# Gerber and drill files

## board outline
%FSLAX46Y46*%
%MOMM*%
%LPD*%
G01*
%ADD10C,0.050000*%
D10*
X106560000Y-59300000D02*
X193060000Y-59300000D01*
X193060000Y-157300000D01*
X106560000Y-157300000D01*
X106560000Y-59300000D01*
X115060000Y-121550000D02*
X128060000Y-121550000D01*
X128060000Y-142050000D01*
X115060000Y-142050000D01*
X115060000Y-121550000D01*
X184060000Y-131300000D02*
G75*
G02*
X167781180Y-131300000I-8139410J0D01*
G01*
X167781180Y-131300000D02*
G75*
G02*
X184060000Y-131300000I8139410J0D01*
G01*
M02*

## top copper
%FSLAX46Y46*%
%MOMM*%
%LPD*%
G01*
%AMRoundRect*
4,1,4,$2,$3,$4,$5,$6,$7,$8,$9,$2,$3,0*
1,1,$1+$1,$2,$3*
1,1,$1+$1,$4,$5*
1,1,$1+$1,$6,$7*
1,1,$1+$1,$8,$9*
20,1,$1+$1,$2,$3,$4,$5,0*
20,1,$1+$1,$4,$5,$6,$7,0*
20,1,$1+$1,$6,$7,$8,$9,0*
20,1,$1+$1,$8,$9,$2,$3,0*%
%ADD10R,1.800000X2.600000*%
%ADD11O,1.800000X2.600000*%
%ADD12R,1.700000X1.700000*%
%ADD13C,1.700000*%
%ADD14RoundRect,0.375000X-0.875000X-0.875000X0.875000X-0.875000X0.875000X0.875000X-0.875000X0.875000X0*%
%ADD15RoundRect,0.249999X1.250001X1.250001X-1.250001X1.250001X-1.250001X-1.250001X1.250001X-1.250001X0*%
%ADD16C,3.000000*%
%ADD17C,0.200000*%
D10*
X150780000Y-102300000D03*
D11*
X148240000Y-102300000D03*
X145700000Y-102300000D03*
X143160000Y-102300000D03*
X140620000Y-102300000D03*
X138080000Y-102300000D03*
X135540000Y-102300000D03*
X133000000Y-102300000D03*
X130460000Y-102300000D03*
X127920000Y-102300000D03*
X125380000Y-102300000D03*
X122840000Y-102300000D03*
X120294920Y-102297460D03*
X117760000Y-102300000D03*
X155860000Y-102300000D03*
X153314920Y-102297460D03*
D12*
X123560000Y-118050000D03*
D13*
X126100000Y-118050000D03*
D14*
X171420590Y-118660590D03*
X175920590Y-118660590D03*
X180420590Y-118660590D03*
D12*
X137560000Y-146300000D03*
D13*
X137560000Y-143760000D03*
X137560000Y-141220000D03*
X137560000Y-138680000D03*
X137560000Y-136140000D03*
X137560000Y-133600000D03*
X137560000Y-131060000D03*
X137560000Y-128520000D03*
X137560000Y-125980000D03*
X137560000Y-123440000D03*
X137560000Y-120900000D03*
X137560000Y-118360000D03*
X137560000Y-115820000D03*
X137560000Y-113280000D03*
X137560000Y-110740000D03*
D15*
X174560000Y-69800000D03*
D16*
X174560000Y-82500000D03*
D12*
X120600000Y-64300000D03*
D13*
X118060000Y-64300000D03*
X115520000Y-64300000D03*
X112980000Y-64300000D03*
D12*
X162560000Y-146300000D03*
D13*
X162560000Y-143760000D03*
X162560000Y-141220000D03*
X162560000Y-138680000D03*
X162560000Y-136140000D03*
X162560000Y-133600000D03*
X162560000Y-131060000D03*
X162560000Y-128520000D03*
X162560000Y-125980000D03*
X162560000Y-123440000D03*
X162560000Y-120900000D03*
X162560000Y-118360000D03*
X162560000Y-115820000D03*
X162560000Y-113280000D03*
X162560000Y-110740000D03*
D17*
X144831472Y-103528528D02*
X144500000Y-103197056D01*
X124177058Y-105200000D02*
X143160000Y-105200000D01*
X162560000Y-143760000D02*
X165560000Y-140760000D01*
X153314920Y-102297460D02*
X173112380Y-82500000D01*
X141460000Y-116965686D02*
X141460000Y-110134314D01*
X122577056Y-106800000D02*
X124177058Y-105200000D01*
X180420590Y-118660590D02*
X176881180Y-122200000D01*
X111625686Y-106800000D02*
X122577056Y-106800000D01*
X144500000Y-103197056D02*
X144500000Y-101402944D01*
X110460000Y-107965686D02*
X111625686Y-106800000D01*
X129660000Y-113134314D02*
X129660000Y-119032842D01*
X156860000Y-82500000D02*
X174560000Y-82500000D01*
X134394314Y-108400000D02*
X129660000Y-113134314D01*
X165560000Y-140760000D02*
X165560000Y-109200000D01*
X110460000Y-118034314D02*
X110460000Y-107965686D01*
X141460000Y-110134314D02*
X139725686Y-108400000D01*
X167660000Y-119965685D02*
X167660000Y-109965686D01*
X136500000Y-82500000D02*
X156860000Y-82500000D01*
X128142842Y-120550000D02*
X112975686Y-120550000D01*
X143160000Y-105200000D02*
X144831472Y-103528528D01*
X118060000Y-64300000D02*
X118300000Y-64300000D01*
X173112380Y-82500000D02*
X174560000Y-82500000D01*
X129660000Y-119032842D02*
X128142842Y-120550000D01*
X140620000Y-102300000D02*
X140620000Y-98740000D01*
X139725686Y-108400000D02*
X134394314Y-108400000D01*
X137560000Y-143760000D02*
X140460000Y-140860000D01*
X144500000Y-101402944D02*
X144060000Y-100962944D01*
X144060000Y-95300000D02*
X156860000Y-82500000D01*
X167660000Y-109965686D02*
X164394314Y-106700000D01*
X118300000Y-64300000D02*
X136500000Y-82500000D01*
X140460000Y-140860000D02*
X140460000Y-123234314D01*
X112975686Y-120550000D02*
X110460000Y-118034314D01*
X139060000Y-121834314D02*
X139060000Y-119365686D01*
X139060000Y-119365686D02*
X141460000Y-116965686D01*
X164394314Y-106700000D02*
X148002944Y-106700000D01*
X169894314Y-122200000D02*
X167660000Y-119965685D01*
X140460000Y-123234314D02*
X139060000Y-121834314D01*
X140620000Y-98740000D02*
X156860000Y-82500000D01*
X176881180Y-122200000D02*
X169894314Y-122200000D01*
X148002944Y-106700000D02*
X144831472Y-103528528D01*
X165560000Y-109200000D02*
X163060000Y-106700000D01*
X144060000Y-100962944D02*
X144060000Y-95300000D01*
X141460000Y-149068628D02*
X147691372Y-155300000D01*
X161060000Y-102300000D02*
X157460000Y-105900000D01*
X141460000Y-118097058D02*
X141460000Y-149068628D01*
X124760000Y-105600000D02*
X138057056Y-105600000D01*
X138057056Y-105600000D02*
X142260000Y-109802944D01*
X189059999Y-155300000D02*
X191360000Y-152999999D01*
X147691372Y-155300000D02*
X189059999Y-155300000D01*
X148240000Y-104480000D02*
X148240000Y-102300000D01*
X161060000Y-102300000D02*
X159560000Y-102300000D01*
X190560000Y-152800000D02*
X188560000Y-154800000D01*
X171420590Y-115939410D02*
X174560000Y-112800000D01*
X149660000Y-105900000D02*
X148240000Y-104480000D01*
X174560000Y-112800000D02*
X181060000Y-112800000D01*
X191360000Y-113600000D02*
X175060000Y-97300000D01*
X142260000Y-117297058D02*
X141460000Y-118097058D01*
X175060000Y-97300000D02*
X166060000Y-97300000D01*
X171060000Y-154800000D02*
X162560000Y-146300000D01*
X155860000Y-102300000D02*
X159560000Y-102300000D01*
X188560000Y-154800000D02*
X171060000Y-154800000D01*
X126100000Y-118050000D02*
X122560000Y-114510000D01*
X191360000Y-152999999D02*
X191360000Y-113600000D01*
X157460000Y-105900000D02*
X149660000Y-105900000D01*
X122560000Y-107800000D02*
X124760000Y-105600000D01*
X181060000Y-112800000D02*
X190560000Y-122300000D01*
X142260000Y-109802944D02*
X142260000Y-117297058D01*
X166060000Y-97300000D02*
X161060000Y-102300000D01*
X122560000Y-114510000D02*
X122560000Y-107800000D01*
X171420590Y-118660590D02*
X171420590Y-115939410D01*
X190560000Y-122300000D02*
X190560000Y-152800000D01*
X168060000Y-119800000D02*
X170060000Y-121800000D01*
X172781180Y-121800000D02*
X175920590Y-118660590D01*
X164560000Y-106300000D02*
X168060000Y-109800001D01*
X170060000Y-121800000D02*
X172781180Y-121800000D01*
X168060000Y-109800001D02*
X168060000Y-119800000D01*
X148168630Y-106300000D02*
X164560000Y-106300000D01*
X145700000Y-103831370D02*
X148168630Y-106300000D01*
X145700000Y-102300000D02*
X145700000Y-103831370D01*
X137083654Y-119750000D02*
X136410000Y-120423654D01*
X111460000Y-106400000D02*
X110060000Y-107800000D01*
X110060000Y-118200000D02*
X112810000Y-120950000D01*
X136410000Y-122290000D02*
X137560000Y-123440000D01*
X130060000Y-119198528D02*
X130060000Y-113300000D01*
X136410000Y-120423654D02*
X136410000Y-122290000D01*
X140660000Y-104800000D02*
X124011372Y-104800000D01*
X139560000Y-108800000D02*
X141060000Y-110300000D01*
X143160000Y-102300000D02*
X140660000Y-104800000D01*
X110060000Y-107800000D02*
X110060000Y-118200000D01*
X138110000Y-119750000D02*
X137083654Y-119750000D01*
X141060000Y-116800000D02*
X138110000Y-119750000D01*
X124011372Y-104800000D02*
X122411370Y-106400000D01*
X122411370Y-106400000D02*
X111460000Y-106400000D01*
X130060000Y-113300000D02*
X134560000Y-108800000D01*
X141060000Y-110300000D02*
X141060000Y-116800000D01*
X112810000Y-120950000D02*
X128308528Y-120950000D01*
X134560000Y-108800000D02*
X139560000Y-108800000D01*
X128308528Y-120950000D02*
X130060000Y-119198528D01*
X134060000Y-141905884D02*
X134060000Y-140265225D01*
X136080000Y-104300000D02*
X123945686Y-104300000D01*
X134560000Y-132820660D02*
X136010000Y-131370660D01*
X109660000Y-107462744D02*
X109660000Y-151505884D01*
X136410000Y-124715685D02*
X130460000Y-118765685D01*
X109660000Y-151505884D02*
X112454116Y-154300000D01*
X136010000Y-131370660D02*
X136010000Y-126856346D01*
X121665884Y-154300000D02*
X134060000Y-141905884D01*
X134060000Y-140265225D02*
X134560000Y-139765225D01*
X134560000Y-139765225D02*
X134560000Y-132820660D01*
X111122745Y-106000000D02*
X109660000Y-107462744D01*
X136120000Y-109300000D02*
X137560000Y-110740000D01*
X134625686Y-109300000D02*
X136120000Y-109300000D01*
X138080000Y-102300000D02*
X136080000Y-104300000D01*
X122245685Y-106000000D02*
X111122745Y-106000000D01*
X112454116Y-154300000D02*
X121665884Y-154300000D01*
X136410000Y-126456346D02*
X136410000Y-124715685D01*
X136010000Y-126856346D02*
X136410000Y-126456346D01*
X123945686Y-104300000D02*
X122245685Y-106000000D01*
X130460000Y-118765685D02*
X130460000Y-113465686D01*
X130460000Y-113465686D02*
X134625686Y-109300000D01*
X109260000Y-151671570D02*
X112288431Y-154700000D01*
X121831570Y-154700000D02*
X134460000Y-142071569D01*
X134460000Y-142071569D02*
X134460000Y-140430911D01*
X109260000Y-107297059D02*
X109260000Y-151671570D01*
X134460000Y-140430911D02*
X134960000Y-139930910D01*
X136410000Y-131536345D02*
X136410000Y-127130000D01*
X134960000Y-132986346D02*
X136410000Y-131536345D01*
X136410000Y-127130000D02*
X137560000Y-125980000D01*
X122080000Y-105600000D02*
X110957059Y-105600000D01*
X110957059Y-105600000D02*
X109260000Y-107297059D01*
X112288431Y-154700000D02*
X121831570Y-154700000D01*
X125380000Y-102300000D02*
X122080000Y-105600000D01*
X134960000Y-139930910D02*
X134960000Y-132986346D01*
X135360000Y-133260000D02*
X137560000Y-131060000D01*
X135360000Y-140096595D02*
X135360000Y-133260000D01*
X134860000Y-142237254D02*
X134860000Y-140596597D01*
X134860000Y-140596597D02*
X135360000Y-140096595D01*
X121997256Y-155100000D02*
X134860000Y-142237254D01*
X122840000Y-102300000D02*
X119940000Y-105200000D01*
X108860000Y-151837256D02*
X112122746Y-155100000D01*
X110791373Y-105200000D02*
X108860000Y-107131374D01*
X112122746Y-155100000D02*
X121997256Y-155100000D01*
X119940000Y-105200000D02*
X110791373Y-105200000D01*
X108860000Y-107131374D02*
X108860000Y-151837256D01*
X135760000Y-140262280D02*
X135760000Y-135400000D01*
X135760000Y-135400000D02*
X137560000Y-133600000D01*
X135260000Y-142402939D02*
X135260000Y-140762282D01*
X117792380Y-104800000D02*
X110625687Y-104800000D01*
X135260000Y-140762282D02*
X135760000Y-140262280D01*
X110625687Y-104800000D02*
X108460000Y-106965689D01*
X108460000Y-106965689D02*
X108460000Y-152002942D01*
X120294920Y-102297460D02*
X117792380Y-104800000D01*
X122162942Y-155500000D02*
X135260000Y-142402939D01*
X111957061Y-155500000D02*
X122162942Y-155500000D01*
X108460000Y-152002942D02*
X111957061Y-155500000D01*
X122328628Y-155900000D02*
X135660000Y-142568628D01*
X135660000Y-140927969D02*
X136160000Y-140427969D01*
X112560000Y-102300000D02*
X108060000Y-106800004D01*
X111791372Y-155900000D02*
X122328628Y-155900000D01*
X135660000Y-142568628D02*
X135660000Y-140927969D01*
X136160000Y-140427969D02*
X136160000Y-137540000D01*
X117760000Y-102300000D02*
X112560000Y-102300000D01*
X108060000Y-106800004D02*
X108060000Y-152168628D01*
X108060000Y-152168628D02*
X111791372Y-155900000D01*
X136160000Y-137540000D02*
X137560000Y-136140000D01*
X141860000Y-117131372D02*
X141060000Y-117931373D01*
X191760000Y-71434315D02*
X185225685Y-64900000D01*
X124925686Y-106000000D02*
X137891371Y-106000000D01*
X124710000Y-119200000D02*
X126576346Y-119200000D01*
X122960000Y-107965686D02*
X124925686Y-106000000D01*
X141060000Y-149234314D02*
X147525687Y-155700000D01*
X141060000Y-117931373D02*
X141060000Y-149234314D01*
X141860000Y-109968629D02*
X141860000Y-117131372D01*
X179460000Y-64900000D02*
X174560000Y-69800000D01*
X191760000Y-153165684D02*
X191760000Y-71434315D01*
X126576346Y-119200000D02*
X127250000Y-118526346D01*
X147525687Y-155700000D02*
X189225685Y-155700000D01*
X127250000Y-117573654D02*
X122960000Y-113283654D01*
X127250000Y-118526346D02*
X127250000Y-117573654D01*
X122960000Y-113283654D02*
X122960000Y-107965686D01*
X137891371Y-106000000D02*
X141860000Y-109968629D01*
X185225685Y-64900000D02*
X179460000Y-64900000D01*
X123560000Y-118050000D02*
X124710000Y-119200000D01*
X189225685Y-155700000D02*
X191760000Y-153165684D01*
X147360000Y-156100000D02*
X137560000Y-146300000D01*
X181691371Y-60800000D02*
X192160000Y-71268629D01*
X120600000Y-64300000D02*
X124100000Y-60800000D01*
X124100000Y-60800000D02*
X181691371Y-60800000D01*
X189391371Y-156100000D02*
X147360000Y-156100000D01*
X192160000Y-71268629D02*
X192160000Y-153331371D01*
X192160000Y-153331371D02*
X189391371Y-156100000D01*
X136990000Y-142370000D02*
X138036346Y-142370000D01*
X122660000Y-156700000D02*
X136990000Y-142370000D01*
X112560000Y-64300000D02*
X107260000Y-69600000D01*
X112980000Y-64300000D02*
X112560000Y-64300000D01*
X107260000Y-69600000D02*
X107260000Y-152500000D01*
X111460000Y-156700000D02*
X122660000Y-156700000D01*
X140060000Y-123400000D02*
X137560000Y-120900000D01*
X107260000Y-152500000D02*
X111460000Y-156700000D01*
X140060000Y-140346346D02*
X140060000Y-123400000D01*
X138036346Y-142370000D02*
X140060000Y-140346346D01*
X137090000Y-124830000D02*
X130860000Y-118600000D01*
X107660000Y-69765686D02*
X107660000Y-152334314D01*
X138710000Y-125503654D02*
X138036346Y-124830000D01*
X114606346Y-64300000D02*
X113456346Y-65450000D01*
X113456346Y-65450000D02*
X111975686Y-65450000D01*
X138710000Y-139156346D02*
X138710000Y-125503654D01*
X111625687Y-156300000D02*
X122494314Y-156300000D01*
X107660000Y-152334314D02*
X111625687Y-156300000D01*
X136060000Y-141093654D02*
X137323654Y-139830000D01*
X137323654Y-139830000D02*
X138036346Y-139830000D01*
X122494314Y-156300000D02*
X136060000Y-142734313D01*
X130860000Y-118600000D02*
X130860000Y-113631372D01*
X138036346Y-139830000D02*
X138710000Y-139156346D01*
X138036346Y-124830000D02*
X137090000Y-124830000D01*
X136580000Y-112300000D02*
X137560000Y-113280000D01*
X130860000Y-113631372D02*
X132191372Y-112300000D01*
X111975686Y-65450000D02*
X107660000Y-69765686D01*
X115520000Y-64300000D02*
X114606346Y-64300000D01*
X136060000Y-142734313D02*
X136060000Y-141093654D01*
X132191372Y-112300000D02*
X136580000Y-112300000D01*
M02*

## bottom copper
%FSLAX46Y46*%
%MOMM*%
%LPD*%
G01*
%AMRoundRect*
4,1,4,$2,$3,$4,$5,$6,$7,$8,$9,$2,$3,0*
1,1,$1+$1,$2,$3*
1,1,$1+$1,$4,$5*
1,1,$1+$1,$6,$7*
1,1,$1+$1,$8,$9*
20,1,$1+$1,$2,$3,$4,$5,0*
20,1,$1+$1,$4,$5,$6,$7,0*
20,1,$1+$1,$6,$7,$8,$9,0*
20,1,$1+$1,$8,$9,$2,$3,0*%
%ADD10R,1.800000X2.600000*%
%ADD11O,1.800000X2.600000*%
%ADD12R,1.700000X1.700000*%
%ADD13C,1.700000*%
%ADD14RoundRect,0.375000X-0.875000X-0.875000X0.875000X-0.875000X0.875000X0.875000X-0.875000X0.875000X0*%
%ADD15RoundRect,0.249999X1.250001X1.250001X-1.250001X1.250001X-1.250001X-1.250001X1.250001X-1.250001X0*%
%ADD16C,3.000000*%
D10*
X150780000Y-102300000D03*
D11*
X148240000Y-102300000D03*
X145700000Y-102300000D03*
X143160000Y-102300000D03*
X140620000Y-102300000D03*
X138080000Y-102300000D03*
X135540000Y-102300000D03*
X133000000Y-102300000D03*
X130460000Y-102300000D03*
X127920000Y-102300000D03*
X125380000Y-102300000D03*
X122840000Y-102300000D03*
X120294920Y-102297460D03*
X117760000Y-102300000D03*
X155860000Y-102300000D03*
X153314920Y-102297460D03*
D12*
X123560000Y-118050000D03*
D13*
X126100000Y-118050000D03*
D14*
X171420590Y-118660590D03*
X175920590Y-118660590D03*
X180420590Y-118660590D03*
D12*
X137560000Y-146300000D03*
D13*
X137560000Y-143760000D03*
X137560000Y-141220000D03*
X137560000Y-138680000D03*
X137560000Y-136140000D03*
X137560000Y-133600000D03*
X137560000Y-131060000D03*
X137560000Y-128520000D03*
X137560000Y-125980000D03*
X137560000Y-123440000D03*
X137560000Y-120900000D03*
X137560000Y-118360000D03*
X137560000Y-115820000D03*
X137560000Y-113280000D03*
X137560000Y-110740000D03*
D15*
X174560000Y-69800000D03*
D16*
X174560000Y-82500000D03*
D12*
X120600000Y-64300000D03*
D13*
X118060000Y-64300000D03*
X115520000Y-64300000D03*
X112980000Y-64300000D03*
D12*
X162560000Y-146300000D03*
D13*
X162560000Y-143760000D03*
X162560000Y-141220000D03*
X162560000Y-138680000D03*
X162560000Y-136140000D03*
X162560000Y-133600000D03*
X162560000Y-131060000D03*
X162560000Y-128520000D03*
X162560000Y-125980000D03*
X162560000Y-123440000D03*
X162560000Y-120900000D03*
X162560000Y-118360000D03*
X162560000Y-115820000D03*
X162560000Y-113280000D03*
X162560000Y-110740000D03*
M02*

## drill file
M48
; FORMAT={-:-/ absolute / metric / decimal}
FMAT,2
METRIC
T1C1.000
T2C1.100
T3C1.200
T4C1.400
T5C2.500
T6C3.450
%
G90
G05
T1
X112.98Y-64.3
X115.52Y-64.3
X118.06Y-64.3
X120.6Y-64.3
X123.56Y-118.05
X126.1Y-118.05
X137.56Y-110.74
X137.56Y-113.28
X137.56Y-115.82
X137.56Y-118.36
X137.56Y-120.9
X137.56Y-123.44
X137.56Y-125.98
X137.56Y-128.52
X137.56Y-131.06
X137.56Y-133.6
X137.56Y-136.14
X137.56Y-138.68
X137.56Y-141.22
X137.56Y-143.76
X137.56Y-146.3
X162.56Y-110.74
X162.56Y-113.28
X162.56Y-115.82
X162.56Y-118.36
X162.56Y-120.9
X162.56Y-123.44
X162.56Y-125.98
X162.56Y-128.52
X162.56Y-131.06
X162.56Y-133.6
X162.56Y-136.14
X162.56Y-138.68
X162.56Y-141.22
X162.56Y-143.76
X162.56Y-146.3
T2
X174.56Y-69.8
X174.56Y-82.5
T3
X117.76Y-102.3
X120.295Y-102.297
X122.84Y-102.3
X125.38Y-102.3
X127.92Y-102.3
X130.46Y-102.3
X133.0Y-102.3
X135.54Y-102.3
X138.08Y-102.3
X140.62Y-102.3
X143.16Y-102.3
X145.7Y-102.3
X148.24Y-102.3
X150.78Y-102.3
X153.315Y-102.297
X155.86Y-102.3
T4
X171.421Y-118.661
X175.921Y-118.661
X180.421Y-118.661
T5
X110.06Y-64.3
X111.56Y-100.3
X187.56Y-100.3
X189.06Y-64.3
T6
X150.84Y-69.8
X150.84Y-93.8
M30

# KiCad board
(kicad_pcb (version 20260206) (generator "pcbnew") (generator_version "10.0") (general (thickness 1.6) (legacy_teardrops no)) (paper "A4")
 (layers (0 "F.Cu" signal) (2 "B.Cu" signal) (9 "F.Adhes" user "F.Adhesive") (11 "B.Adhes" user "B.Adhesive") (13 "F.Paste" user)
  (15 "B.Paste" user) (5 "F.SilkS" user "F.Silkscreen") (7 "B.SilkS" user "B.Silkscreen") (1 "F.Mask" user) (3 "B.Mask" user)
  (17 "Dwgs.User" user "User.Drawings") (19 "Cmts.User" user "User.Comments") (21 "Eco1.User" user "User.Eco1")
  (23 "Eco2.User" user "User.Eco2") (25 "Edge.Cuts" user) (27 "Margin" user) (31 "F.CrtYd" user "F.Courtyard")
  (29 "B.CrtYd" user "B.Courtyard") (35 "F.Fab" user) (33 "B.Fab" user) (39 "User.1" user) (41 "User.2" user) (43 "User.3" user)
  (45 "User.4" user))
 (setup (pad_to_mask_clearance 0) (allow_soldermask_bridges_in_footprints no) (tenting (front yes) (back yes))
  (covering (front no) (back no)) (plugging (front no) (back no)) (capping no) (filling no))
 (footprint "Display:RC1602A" (layer "F.Cu") (at 150.78 102.3 180)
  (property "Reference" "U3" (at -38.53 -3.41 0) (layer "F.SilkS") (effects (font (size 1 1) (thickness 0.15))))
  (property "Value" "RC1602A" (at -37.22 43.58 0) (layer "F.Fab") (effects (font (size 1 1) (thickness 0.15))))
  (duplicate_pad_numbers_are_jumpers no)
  (pad "" np_thru_hole circle (at -38.28 38) (size 2.5 2.5) (drill 2.5) (layers "*.Cu" "*.Mask"))
  (pad "" np_thru_hole circle (at -36.78 2) (size 2.5 2.5) (drill 2.5) (layers "*.Cu" "*.Mask"))
  (pad "" np_thru_hole circle (at 39.22 2) (size 2.5 2.5) (drill 2.5) (layers "*.Cu" "*.Mask"))
  (pad "" np_thru_hole circle (at 40.72 38) (size 2.5 2.5) (drill 2.5) (layers "*.Cu" "*.Mask"))
  (pad "1" thru_hole rect (at 0 0) (size 1.8 2.6) (drill 1.2) (layers "*.Cu" "*.Mask") (remove_unused_layers no) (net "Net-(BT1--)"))
  (pad "2" thru_hole oval (at 2.54 0) (size 1.8 2.6) (drill 1.2) (layers "*.Cu" "*.Mask") (remove_unused_layers no) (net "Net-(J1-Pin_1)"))
  (pad "3" thru_hole oval (at 5.08 0) (size 1.8 2.6) (drill 1.2) (layers "*.Cu" "*.Mask") (remove_unused_layers no) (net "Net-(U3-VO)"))
  (pad "4" thru_hole oval (at 7.62 0) (size 1.8 2.6) (drill 1.2) (layers "*.Cu" "*.Mask") (remove_unused_layers no) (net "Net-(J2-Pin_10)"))
  (pad "5" thru_hole oval (at 10.16 0) (size 1.8 2.6) (drill 1.2) (layers "*.Cu" "*.Mask") (remove_unused_layers no) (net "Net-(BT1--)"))
  (pad "6" thru_hole oval (at 12.7 0) (size 1.8 2.6) (drill 1.2) (layers "*.Cu" "*.Mask") (remove_unused_layers no) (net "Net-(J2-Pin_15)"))
  (pad "7" thru_hole oval (at 15.24 0) (size 1.8 2.6) (drill 1.2) (layers "*.Cu" "*.Mask") (remove_unused_layers no)
   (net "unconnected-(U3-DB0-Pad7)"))
  (pad "8" thru_hole oval (at 17.78 0) (size 1.8 2.6) (drill 1.2) (layers "*.Cu" "*.Mask") (remove_unused_layers no)
   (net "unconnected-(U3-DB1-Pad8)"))
  (pad "9" thru_hole oval (at 20.32 0) (size 1.8 2.6) (drill 1.2) (layers "*.Cu" "*.Mask") (remove_unused_layers no)
   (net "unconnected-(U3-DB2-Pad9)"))
  (pad "10" thru_hole oval (at 22.86 0) (size 1.8 2.6) (drill 1.2) (layers "*.Cu" "*.Mask") (remove_unused_layers no)
   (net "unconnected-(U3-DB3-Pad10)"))
  (pad "11" thru_hole oval (at 25.4 0) (size 1.8 2.6) (drill 1.2) (layers "*.Cu" "*.Mask") (remove_unused_layers no) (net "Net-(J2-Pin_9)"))
  (pad "12" thru_hole oval (at 27.94 0) (size 1.8 2.6) (drill 1.2) (layers "*.Cu" "*.Mask") (remove_unused_layers no) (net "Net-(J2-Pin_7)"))
  (pad "13" thru_hole oval (at 30.48508 0.00254) (size 1.8 2.6) (drill 1.2) (layers "*.Cu" "*.Mask") (remove_unused_layers no)
   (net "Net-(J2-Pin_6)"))
  (pad "14" thru_hole oval (at 33.02 0) (size 1.8 2.6) (drill 1.2) (layers "*.Cu" "*.Mask") (remove_unused_layers no) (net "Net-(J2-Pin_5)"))
  (pad "15" thru_hole oval (at -5.08 0) (size 1.8 2.6) (drill 1.2) (layers "*.Cu" "*.Mask") (remove_unused_layers no) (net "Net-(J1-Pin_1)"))
  (pad "16" thru_hole oval (at -2.53492 0.00254) (size 1.8 2.6) (drill 1.2) (layers "*.Cu" "*.Mask") (remove_unused_layers no)
   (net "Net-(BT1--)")))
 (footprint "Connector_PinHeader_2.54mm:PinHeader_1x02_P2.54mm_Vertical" (layer "F.Cu") (at 123.56 118.05 90)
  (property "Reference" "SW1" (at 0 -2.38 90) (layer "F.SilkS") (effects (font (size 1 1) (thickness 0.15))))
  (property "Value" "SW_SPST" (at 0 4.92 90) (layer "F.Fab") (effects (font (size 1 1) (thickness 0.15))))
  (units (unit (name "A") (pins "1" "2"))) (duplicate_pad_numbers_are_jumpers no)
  (pad "1" thru_hole rect (at 0 0 90) (size 1.7 1.7) (drill 1) (layers "*.Cu" "*.Mask") (remove_unused_layers no) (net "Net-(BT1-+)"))
  (pad "2" thru_hole circle (at 0 2.54 90) (size 1.7 1.7) (drill 1) (layers "*.Cu" "*.Mask") (remove_unused_layers no)
   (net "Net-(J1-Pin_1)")))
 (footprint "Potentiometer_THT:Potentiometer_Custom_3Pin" (layer "F.Cu") (at 175.92059 118.66059)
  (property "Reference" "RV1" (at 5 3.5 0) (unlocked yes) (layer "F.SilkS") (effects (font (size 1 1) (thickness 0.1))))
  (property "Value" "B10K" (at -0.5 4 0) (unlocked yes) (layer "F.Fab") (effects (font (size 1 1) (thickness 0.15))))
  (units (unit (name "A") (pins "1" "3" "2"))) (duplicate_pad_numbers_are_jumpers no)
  (pad "1" thru_hole roundrect (at -4.5 0) (size 2.5 2.5) (drill 1.4) (layers "*.Cu" "*.Mask") (remove_unused_layers no)
   (roundrect_rratio 0.15) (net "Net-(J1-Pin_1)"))
  (pad "2" thru_hole roundrect (at 0 0) (size 2.5 2.5) (drill 1.4) (layers "*.Cu" "*.Mask") (remove_unused_layers no)
   (roundrect_rratio 0.15) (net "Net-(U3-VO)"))
  (pad "3" thru_hole roundrect (at 4.5 0) (size 2.5 2.5) (drill 1.4) (layers "*.Cu" "*.Mask") (remove_unused_layers no)
   (roundrect_rratio 0.15) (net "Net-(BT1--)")))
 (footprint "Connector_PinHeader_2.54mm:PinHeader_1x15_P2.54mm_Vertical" (layer "B.Cu") (at 137.56 146.3)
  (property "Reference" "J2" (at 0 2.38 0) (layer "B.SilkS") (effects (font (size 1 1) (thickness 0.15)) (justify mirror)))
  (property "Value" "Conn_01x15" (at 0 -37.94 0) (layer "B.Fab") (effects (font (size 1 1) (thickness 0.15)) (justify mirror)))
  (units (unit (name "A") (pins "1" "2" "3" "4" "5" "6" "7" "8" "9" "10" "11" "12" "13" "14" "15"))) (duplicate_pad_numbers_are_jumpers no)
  (pad "1" thru_hole rect (at 0 0) (size 1.7 1.7) (drill 1) (layers "*.Cu" "*.Mask") (remove_unused_layers no) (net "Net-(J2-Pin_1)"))
  (pad "2" thru_hole circle (at 0 -2.54) (size 1.7 1.7) (drill 1) (layers "*.Cu" "*.Mask") (remove_unused_layers no) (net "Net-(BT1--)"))
  (pad "3" thru_hole circle (at 0 -5.08) (size 1.7 1.7) (drill 1) (layers "*.Cu" "*.Mask") (remove_unused_layers no)
   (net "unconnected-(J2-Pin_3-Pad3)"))
  (pad "4" thru_hole circle (at 0 -7.62) (size 1.7 1.7) (drill 1) (layers "*.Cu" "*.Mask") (remove_unused_layers no)
   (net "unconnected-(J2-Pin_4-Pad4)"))
  (pad "5" thru_hole circle (at 0 -10.16) (size 1.7 1.7) (drill 1) (layers "*.Cu" "*.Mask") (remove_unused_layers no) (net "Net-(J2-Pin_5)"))
  (pad "6" thru_hole circle (at 0 -12.7) (size 1.7 1.7) (drill 1) (layers "*.Cu" "*.Mask") (remove_unused_layers no) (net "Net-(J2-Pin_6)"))
  (pad "7" thru_hole circle (at 0 -15.24) (size 1.7 1.7) (drill 1) (layers "*.Cu" "*.Mask") (remove_unused_layers no) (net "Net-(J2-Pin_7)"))
  (pad "8" thru_hole circle (at 0 -17.78) (size 1.7 1.7) (drill 1) (layers "*.Cu" "*.Mask") (remove_unused_layers no)
   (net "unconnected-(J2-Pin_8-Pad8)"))
  (pad "9" thru_hole circle (at 0 -20.32) (size 1.7 1.7) (drill 1) (layers "*.Cu" "*.Mask") (remove_unused_layers no) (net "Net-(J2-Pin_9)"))
  (pad "10" thru_hole circle (at 0 -22.86) (size 1.7 1.7) (drill 1) (layers "*.Cu" "*.Mask") (remove_unused_layers no)
   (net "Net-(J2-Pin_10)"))
  (pad "11" thru_hole circle (at 0 -25.4) (size 1.7 1.7) (drill 1) (layers "*.Cu" "*.Mask") (remove_unused_layers no)
   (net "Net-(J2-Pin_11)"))
  (pad "12" thru_hole circle (at 0 -27.94) (size 1.7 1.7) (drill 1) (layers "*.Cu" "*.Mask") (remove_unused_layers no)
   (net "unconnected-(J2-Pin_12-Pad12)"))
  (pad "13" thru_hole circle (at 0 -30.48) (size 1.7 1.7) (drill 1) (layers "*.Cu" "*.Mask") (remove_unused_layers no)
   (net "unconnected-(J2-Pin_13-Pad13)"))
  (pad "14" thru_hole circle (at 0 -33.02) (size 1.7 1.7) (drill 1) (layers "*.Cu" "*.Mask") (remove_unused_layers no)
   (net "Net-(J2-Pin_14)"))
  (pad "15" thru_hole circle (at 0 -35.56) (size 1.7 1.7) (drill 1) (layers "*.Cu" "*.Mask") (remove_unused_layers no)
   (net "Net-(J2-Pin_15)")))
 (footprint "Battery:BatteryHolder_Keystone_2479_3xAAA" (layer "B.Cu") (at 174.56 69.8 180)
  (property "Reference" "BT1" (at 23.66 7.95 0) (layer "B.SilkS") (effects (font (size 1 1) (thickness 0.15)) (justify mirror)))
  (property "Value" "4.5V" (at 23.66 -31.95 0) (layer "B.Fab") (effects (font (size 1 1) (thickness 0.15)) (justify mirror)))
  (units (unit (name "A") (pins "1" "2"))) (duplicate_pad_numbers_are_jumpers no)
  (pad "" np_thru_hole circle (at 23.72 -24 180) (size 3.45 3.45) (drill 3.45) (layers "*.Cu" "*.Mask"))
  (pad "" np_thru_hole circle (at 23.72 0 180) (size 3.45 3.45) (drill 3.45) (layers "*.Cu" "*.Mask"))
  (pad "1" thru_hole roundrect (at 0 0 180) (size 3 3) (drill 1.1) (layers "*.Cu" "*.Mask") (remove_unused_layers no)
   (roundrect_rratio 0.083333) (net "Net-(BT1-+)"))
  (pad "2" thru_hole circle (at 0 -12.7 180) (size 3 3) (drill 1.1) (layers "*.Cu" "*.Mask") (remove_unused_layers no) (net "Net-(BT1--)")))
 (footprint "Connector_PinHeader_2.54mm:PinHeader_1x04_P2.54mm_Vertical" (layer "B.Cu") (at 120.6 64.3 90)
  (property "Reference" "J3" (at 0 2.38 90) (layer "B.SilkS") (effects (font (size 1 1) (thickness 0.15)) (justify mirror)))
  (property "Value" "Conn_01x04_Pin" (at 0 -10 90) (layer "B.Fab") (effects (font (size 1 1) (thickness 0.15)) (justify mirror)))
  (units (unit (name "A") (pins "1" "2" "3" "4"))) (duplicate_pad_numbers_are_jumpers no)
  (pad "1" thru_hole rect (at 0 0 90) (size 1.7 1.7) (drill 1) (layers "*.Cu" "*.Mask") (remove_unused_layers no) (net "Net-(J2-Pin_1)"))
  (pad "2" thru_hole circle (at 0 -2.54 90) (size 1.7 1.7) (drill 1) (layers "*.Cu" "*.Mask") (remove_unused_layers no) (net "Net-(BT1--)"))
  (pad "3" thru_hole circle (at 0 -5.08 90) (size 1.7 1.7) (drill 1) (layers "*.Cu" "*.Mask") (remove_unused_layers no)
   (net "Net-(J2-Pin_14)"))
  (pad "4" thru_hole circle (at 0 -7.62 90) (size 1.7 1.7) (drill 1) (layers "*.Cu" "*.Mask") (remove_unused_layers no)
   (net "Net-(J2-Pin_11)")))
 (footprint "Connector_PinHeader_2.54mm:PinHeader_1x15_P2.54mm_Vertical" (layer "B.Cu") (at 162.56 146.3)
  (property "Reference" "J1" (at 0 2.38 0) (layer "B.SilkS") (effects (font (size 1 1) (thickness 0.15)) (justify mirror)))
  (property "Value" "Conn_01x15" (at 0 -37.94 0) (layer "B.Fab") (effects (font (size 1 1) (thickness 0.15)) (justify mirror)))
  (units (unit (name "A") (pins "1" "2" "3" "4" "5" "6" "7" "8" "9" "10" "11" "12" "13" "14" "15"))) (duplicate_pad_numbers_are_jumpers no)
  (pad "1" thru_hole rect (at 0 0) (size 1.7 1.7) (drill 1) (layers "*.Cu" "*.Mask") (remove_unused_layers no) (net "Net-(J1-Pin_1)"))
  (pad "2" thru_hole circle (at 0 -2.54) (size 1.7 1.7) (drill 1) (layers "*.Cu" "*.Mask") (remove_unused_layers no) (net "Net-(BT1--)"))
  (pad "3" thru_hole circle (at 0 -5.08) (size 1.7 1.7) (drill 1) (layers "*.Cu" "*.Mask") (remove_unused_layers no)
   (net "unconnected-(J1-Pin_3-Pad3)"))
  (pad "4" thru_hole circle (at 0 -7.62) (size 1.7 1.7) (drill 1) (layers "*.Cu" "*.Mask") (remove_unused_layers no)
   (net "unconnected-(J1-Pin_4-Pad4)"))
  (pad "5" thru_hole circle (at 0 -10.16) (size 1.7 1.7) (drill 1) (layers "*.Cu" "*.Mask") (remove_unused_layers no)
   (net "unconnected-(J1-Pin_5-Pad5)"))
  (pad "6" thru_hole circle (at 0 -12.7) (size 1.7 1.7) (drill 1) (layers "*.Cu" "*.Mask") (remove_unused_layers no)
   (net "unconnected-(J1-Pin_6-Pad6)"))
  (pad "7" thru_hole circle (at 0 -15.24) (size 1.7 1.7) (drill 1) (layers "*.Cu" "*.Mask") (remove_unused_layers no)
   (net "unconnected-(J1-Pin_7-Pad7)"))
  (pad "8" thru_hole circle (at 0 -17.78) (size 1.7 1.7) (drill 1) (layers "*.Cu" "*.Mask") (remove_unused_layers no)
   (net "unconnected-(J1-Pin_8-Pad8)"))
  (pad "9" thru_hole circle (at 0 -20.32) (size 1.7 1.7) (drill 1) (layers "*.Cu" "*.Mask") (remove_unused_layers no)
   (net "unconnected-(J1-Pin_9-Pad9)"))
  (pad "10" thru_hole circle (at 0 -22.86) (size 1.7 1.7) (drill 1) (layers "*.Cu" "*.Mask") (remove_unused_layers no)
   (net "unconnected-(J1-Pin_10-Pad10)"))
  (pad "11" thru_hole circle (at 0 -25.4) (size 1.7 1.7) (drill 1) (layers "*.Cu" "*.Mask") (remove_unused_layers no)
   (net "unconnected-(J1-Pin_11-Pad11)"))
  (pad "12" thru_hole circle (at 0 -27.94) (size 1.7 1.7) (drill 1) (layers "*.Cu" "*.Mask") (remove_unused_layers no)
   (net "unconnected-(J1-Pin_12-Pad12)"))
  (pad "13" thru_hole circle (at 0 -30.48) (size 1.7 1.7) (drill 1) (layers "*.Cu" "*.Mask") (remove_unused_layers no)
   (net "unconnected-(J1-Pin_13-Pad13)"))
  (pad "14" thru_hole circle (at 0 -33.02) (size 1.7 1.7) (drill 1) (layers "*.Cu" "*.Mask") (remove_unused_layers no)
   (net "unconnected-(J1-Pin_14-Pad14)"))
  (pad "15" thru_hole circle (at 0 -35.56) (size 1.7 1.7) (drill 1) (layers "*.Cu" "*.Mask") (remove_unused_layers no)
   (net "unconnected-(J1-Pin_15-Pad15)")))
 (gr_rect (start 106.56 59.3) (end 193.06 157.3) (stroke (width 0.05) (type default)) (fill no) (layer "Edge.Cuts"))
 (gr_rect (start 115.06 121.55) (end 128.06 142.05) (stroke (width 0.05) (type default)) (fill no) (layer "Edge.Cuts"))
 (gr_circle (center 175.92059 131.3) (end 181.92059 136.8) (stroke (width 0.05) (type solid)) (fill no) (layer "Edge.Cuts"))
 (segment (start 144.831472 103.528528) (end 144.5 103.197056) (width 0.2) (layer "F.Cu") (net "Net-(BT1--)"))
 (segment (start 124.177058 105.2) (end 143.16 105.2) (width 0.2) (layer "F.Cu") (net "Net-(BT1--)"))
 (segment (start 162.56 143.76) (end 165.56 140.76) (width 0.2) (layer "F.Cu") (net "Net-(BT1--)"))
 (segment (start 153.31492 102.29746) (end 173.11238 82.5) (width 0.2) (layer "F.Cu") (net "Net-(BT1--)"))
 (segment (start 141.46 116.965686) (end 141.46 110.134314) (width 0.2) (layer "F.Cu") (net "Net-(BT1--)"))
 (segment (start 122.577056 106.8) (end 124.177058 105.2) (width 0.2) (layer "F.Cu") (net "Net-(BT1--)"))
 (segment (start 180.42059 118.66059) (end 176.88118 122.2) (width 0.2) (layer "F.Cu") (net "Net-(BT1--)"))
 (segment (start 111.625686 106.8) (end 122.577056 106.8) (width 0.2) (layer "F.Cu") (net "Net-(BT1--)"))
 (segment (start 144.5 103.197056) (end 144.5 101.402944) (width 0.2) (layer "F.Cu") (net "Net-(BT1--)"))
 (segment (start 110.46 107.965686) (end 111.625686 106.8) (width 0.2) (layer "F.Cu") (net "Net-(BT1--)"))
 (segment (start 129.66 113.134314) (end 129.66 119.032842) (width 0.2) (layer "F.Cu") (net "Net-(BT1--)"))
 (segment (start 156.86 82.5) (end 174.56 82.5) (width 0.2) (layer "F.Cu") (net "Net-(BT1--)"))
 (segment (start 134.394314 108.4) (end 129.66 113.134314) (width 0.2) (layer "F.Cu") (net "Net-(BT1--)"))
 (segment (start 165.56 140.76) (end 165.56 109.2) (width 0.2) (layer "F.Cu") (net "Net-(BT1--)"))
 (segment (start 110.46 118.034314) (end 110.46 107.965686) (width 0.2) (layer "F.Cu") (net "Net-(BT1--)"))
 (segment (start 141.46 110.134314) (end 139.725686 108.4) (width 0.2) (layer "F.Cu") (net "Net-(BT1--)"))
 (segment (start 167.66 119.965685) (end 167.66 109.965686) (width 0.2) (layer "F.Cu") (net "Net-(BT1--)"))
 (segment (start 136.5 82.5) (end 156.86 82.5) (width 0.2) (layer "F.Cu") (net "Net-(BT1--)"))
 (segment (start 128.142842 120.55) (end 112.975686 120.55) (width 0.2) (layer "F.Cu") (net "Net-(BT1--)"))
 (segment (start 143.16 105.2) (end 144.831472 103.528528) (width 0.2) (layer "F.Cu") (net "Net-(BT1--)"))
 (segment (start 118.06 64.3) (end 118.3 64.3) (width 0.2) (layer "F.Cu") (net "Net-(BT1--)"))
 (segment (start 173.11238 82.5) (end 174.56 82.5) (width 0.2) (layer "F.Cu") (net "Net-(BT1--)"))
 (segment (start 129.66 119.032842) (end 128.142842 120.55) (width 0.2) (layer "F.Cu") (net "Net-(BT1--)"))
 (segment (start 140.62 102.3) (end 140.62 98.74) (width 0.2) (layer "F.Cu") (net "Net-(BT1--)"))
 (segment (start 139.725686 108.4) (end 134.394314 108.4) (width 0.2) (layer "F.Cu") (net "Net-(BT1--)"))
 (segment (start 137.56 143.76) (end 140.46 140.86) (width 0.2) (layer "F.Cu") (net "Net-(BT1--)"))
 (segment (start 144.5 101.402944) (end 144.06 100.962944) (width 0.2) (layer "F.Cu") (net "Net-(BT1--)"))
 (segment (start 144.06 95.3) (end 156.86 82.5) (width 0.2) (layer "F.Cu") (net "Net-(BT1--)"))
 (segment (start 167.66 109.965686) (end 164.394314 106.7) (width 0.2) (layer "F.Cu") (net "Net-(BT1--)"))
 (segment (start 118.3 64.3) (end 136.5 82.5) (width 0.2) (layer "F.Cu") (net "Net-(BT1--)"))
 (segment (start 140.46 140.86) (end 140.46 123.234314) (width 0.2) (layer "F.Cu") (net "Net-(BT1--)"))
 (segment (start 112.975686 120.55) (end 110.46 118.034314) (width 0.2) (layer "F.Cu") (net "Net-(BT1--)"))
 (segment (start 139.06 121.834314) (end 139.06 119.365686) (width 0.2) (layer "F.Cu") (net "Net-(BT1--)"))
 (segment (start 139.06 119.365686) (end 141.46 116.965686) (width 0.2) (layer "F.Cu") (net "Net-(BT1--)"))
 (segment (start 164.394314 106.7) (end 148.002944 106.7) (width 0.2) (layer "F.Cu") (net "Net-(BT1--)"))
 (segment (start 169.894314 122.2) (end 167.66 119.965685) (width 0.2) (layer "F.Cu") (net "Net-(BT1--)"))
 (segment (start 140.46 123.234314) (end 139.06 121.834314) (width 0.2) (layer "F.Cu") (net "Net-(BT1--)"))
 (segment (start 140.62 98.74) (end 156.86 82.5) (width 0.2) (layer "F.Cu") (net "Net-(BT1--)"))
 (segment (start 176.88118 122.2) (end 169.894314 122.2) (width 0.2) (layer "F.Cu") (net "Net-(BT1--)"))
 (segment (start 148.002944 106.7) (end 144.831472 103.528528) (width 0.2) (layer "F.Cu") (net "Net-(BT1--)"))
 (segment (start 165.56 109.2) (end 163.06 106.7) (width 0.2) (layer "F.Cu") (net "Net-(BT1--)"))
 (segment (start 144.06 100.962944) (end 144.06 95.3) (width 0.2) (layer "F.Cu") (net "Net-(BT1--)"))
 (segment (start 141.46 149.068628) (end 147.691372 155.3) (width 0.2) (layer "F.Cu") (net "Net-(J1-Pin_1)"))
 (segment (start 161.06 102.3) (end 157.46 105.9) (width 0.2) (layer "F.Cu") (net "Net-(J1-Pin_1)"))
 (segment (start 141.46 118.097058) (end 141.46 149.068628) (width 0.2) (layer "F.Cu") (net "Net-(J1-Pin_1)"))
 (segment (start 124.76 105.6) (end 138.057056 105.6) (width 0.2) (layer "F.Cu") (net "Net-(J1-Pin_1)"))
 (segment (start 138.057056 105.6) (end 142.26 109.802944) (width 0.2) (layer "F.Cu") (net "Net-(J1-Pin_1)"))
 (segment (start 189.059999 155.3) (end 191.36 152.999999) (width 0.2) (layer "F.Cu") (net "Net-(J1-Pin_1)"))
 (segment (start 147.691372 155.3) (end 189.059999 155.3) (width 0.2) (layer "F.Cu") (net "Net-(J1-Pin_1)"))
 (segment (start 148.24 104.48) (end 148.24 102.3) (width 0.2) (layer "F.Cu") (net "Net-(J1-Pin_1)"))
 (segment (start 161.06 102.3) (end 159.56 102.3) (width 0.2) (layer "F.Cu") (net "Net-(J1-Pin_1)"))
 (segment (start 190.56 152.8) (end 188.56 154.8) (width 0.2) (layer "F.Cu") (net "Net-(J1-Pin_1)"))
 (segment (start 171.42059 115.93941) (end 174.56 112.8) (width 0.2) (layer "F.Cu") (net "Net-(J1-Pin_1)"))
 (segment (start 149.66 105.9) (end 148.24 104.48) (width 0.2) (layer "F.Cu") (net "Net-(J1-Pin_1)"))
 (segment (start 174.56 112.8) (end 181.06 112.8) (width 0.2) (layer "F.Cu") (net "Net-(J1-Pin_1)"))
 (segment (start 191.36 113.6) (end 175.06 97.3) (width 0.2) (layer "F.Cu") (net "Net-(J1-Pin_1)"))
 (segment (start 142.26 117.297058) (end 141.46 118.097058) (width 0.2) (layer "F.Cu") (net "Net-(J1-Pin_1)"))
 (segment (start 175.06 97.3) (end 166.06 97.3) (width 0.2) (layer "F.Cu") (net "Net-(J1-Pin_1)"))
 (segment (start 171.06 154.8) (end 162.56 146.3) (width 0.2) (layer "F.Cu") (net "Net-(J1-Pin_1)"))
 (segment (start 155.86 102.3) (end 159.56 102.3) (width 0.2) (layer "F.Cu") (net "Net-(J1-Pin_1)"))
 (segment (start 188.56 154.8) (end 171.06 154.8) (width 0.2) (layer "F.Cu") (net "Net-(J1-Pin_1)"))
 (segment (start 126.1 118.05) (end 122.56 114.51) (width 0.2) (layer "F.Cu") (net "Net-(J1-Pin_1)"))
 (segment (start 191.36 152.999999) (end 191.36 113.6) (width 0.2) (layer "F.Cu") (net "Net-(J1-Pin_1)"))
 (segment (start 157.46 105.9) (end 149.66 105.9) (width 0.2) (layer "F.Cu") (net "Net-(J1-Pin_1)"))
 (segment (start 122.56 107.8) (end 124.76 105.6) (width 0.2) (layer "F.Cu") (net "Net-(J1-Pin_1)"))
 (segment (start 181.06 112.8) (end 190.56 122.3) (width 0.2) (layer "F.Cu") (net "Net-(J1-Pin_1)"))
 (segment (start 142.26 109.802944) (end 142.26 117.297058) (width 0.2) (layer "F.Cu") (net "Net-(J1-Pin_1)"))
 (segment (start 166.06 97.3) (end 161.06 102.3) (width 0.2) (layer "F.Cu") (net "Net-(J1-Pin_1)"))
 (segment (start 122.56 114.51) (end 122.56 107.8) (width 0.2) (layer "F.Cu") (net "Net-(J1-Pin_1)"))
 (segment (start 171.42059 118.66059) (end 171.42059 115.93941) (width 0.2) (layer "F.Cu") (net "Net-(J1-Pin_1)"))
 (segment (start 190.56 122.3) (end 190.56 152.8) (width 0.2) (layer "F.Cu") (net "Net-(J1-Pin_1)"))
 (segment (start 168.06 119.8) (end 170.06 121.8) (width 0.2) (layer "F.Cu") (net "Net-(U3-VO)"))
 (segment (start 172.78118 121.8) (end 175.92059 118.66059) (width 0.2) (layer "F.Cu") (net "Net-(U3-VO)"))
 (segment (start 164.56 106.3) (end 168.06 109.800001) (width 0.2) (layer "F.Cu") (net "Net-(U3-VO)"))
 (segment (start 170.06 121.8) (end 172.78118 121.8) (width 0.2) (layer "F.Cu") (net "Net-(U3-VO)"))
 (segment (start 168.06 109.800001) (end 168.06 119.8) (width 0.2) (layer "F.Cu") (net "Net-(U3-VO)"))
 (segment (start 148.16863 106.3) (end 164.56 106.3) (width 0.2) (layer "F.Cu") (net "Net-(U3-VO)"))
 (segment (start 145.7 103.83137) (end 148.16863 106.3) (width 0.2) (layer "F.Cu") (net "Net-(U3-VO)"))
 (segment (start 145.7 102.3) (end 145.7 103.83137) (width 0.2) (layer "F.Cu") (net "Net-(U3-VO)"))
 (segment (start 137.083654 119.75) (end 136.41 120.423654) (width 0.2) (layer "F.Cu") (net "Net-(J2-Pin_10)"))
 (segment (start 111.46 106.4) (end 110.06 107.8) (width 0.2) (layer "F.Cu") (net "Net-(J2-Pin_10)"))
 (segment (start 110.06 118.2) (end 112.81 120.95) (width 0.2) (layer "F.Cu") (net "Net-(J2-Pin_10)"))
 (segment (start 136.41 122.29) (end 137.56 123.44) (width 0.2) (layer "F.Cu") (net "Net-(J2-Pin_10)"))
 (segment (start 130.06 119.198528) (end 130.06 113.3) (width 0.2) (layer "F.Cu") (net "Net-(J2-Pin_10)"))
 (segment (start 136.41 120.423654) (end 136.41 122.29) (width 0.2) (layer "F.Cu") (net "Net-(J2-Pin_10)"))
 (segment (start 140.66 104.8) (end 124.011372 104.8) (width 0.2) (layer "F.Cu") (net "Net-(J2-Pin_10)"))
 (segment (start 139.56 108.8) (end 141.06 110.3) (width 0.2) (layer "F.Cu") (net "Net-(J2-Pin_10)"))
 (segment (start 143.16 102.3) (end 140.66 104.8) (width 0.2) (layer "F.Cu") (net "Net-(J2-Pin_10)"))
 (segment (start 110.06 107.8) (end 110.06 118.2) (width 0.2) (layer "F.Cu") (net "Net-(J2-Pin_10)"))
 (segment (start 138.11 119.75) (end 137.083654 119.75) (width 0.2) (layer "F.Cu") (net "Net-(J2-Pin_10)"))
 (segment (start 141.06 116.8) (end 138.11 119.75) (width 0.2) (layer "F.Cu") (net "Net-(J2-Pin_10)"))
 (segment (start 124.011372 104.8) (end 122.41137 106.4) (width 0.2) (layer "F.Cu") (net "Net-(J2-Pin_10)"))
 (segment (start 122.41137 106.4) (end 111.46 106.4) (width 0.2) (layer "F.Cu") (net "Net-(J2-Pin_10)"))
 (segment (start 130.06 113.3) (end 134.56 108.8) (width 0.2) (layer "F.Cu") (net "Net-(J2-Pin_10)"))
 (segment (start 141.06 110.3) (end 141.06 116.8) (width 0.2) (layer "F.Cu") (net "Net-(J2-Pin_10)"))
 (segment (start 112.81 120.95) (end 128.308528 120.95) (width 0.2) (layer "F.Cu") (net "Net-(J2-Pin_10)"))
 (segment (start 134.56 108.8) (end 139.56 108.8) (width 0.2) (layer "F.Cu") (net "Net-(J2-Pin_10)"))
 (segment (start 128.308528 120.95) (end 130.06 119.198528) (width 0.2) (layer "F.Cu") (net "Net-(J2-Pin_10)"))
 (segment (start 134.06 141.905884) (end 134.06 140.265225) (width 0.2) (layer "F.Cu") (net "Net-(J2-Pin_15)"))
 (segment (start 136.08 104.3) (end 123.945686 104.3) (width 0.2) (layer "F.Cu") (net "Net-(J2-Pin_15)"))
 (segment (start 134.56 132.82066) (end 136.01 131.37066) (width 0.2) (layer "F.Cu") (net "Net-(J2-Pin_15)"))
 (segment (start 109.66 107.462744) (end 109.66 151.505884) (width 0.2) (layer "F.Cu") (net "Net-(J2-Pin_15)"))
 (segment (start 136.41 124.715685) (end 130.46 118.765685) (width 0.2) (layer "F.Cu") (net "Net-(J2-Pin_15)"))
 (segment (start 109.66 151.505884) (end 112.454116 154.3) (width 0.2) (layer "F.Cu") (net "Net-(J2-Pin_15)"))
 (segment (start 136.01 131.37066) (end 136.01 126.856346) (width 0.2) (layer "F.Cu") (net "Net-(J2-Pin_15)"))
 (segment (start 121.665884 154.3) (end 134.06 141.905884) (width 0.2) (layer "F.Cu") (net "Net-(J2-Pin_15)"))
 (segment (start 134.06 140.265225) (end 134.56 139.765225) (width 0.2) (layer "F.Cu") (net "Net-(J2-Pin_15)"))
 (segment (start 134.56 139.765225) (end 134.56 132.82066) (width 0.2) (layer "F.Cu") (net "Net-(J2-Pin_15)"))
 (segment (start 111.122745 106) (end 109.66 107.462744) (width 0.2) (layer "F.Cu") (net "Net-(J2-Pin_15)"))
 (segment (start 136.12 109.3) (end 137.56 110.74) (width 0.2) (layer "F.Cu") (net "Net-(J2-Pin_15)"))
 (segment (start 134.625686 109.3) (end 136.12 109.3) (width 0.2) (layer "F.Cu") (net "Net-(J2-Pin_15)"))
 (segment (start 138.08 102.3) (end 136.08 104.3) (width 0.2) (layer "F.Cu") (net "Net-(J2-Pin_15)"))
 (segment (start 122.245685 106) (end 111.122745 106) (width 0.2) (layer "F.Cu") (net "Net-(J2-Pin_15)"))
 (segment (start 112.454116 154.3) (end 121.665884 154.3) (width 0.2) (layer "F.Cu") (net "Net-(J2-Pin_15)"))
 (segment (start 136.41 126.456346) (end 136.41 124.715685) (width 0.2) (layer "F.Cu") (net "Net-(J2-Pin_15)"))
 (segment (start 136.01 126.856346) (end 136.41 126.456346) (width 0.2) (layer "F.Cu") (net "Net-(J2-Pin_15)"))
 (segment (start 123.945686 104.3) (end 122.245685 106) (width 0.2) (layer "F.Cu") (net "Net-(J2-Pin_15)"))
 (segment (start 130.46 118.765685) (end 130.46 113.465686) (width 0.2) (layer "F.Cu") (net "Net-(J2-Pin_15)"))
 (segment (start 130.46 113.465686) (end 134.625686 109.3) (width 0.2) (layer "F.Cu") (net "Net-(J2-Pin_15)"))
 (segment (start 109.26 151.67157) (end 112.288431 154.7) (width 0.2) (layer "F.Cu") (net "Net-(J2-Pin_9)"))
 (segment (start 121.83157 154.7) (end 134.46 142.071569) (width 0.2) (layer "F.Cu") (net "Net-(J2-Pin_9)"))
 (segment (start 134.46 142.071569) (end 134.46 140.430911) (width 0.2) (layer "F.Cu") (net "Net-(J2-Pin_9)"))
 (segment (start 109.26 107.297059) (end 109.26 151.67157) (width 0.2) (layer "F.Cu") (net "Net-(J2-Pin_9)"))
 (segment (start 134.46 140.430911) (end 134.96 139.93091) (width 0.2) (layer "F.Cu") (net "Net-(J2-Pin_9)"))
 (segment (start 136.41 131.536345) (end 136.41 127.13) (width 0.2) (layer "F.Cu") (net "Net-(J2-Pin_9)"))
 (segment (start 134.96 132.986346) (end 136.41 131.536345) (width 0.2) (layer "F.Cu") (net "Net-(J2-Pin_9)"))
 (segment (start 136.41 127.13) (end 137.56 125.98) (width 0.2) (layer "F.Cu") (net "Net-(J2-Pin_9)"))
 (segment (start 122.08 105.6) (end 110.957059 105.6) (width 0.2) (layer "F.Cu") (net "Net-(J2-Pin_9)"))
 (segment (start 110.957059 105.6) (end 109.26 107.297059) (width 0.2) (layer "F.Cu") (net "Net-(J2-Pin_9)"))
 (segment (start 112.288431 154.7) (end 121.83157 154.7) (width 0.2) (layer "F.Cu") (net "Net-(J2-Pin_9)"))
 (segment (start 125.38 102.3) (end 122.08 105.6) (width 0.2) (layer "F.Cu") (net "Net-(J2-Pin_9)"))
 (segment (start 134.96 139.93091) (end 134.96 132.986346) (width 0.2) (layer "F.Cu") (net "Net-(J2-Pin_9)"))
 (segment (start 135.36 133.26) (end 137.56 131.06) (width 0.2) (layer "F.Cu") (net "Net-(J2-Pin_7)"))
 (segment (start 135.36 140.096595) (end 135.36 133.26) (width 0.2) (layer "F.Cu") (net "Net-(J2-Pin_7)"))
 (segment (start 134.86 142.237254) (end 134.86 140.596597) (width 0.2) (layer "F.Cu") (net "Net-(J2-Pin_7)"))
 (segment (start 134.86 140.596597) (end 135.36 140.096595) (width 0.2) (layer "F.Cu") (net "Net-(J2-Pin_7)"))
 (segment (start 121.997256 155.1) (end 134.86 142.237254) (width 0.2) (layer "F.Cu") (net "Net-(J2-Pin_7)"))
 (segment (start 122.84 102.3) (end 119.94 105.2) (width 0.2) (layer "F.Cu") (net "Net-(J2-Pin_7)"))
 (segment (start 108.86 151.837256) (end 112.122746 155.1) (width 0.2) (layer "F.Cu") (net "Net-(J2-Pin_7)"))
 (segment (start 110.791373 105.2) (end 108.86 107.131374) (width 0.2) (layer "F.Cu") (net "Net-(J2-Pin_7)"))
 (segment (start 112.122746 155.1) (end 121.997256 155.1) (width 0.2) (layer "F.Cu") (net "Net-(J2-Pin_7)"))
 (segment (start 119.94 105.2) (end 110.791373 105.2) (width 0.2) (layer "F.Cu") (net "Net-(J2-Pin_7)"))
 (segment (start 108.86 107.131374) (end 108.86 151.837256) (width 0.2) (layer "F.Cu") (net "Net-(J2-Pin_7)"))
 (segment (start 135.76 140.26228) (end 135.76 135.4) (width 0.2) (layer "F.Cu") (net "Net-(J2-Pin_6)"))
 (segment (start 135.76 135.4) (end 137.56 133.6) (width 0.2) (layer "F.Cu") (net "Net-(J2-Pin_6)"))
 (segment (start 135.26 142.402939) (end 135.26 140.762282) (width 0.2) (layer "F.Cu") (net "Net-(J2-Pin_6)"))
 (segment (start 117.79238 104.8) (end 110.625687 104.8) (width 0.2) (layer "F.Cu") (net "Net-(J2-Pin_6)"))
 (segment (start 135.26 140.762282) (end 135.76 140.26228) (width 0.2) (layer "F.Cu") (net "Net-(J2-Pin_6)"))
 (segment (start 110.625687 104.8) (end 108.46 106.965689) (width 0.2) (layer "F.Cu") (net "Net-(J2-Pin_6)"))
 (segment (start 108.46 106.965689) (end 108.46 152.002942) (width 0.2) (layer "F.Cu") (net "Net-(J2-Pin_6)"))
 (segment (start 120.29492 102.29746) (end 117.79238 104.8) (width 0.2) (layer "F.Cu") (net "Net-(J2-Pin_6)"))
 (segment (start 122.162942 155.5) (end 135.26 142.402939) (width 0.2) (layer "F.Cu") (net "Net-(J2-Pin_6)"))
 (segment (start 111.957061 155.5) (end 122.162942 155.5) (width 0.2) (layer "F.Cu") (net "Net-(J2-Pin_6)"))
 (segment (start 108.46 152.002942) (end 111.957061 155.5) (width 0.2) (layer "F.Cu") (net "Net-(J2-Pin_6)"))
 (segment (start 122.328628 155.9) (end 135.66 142.568628) (width 0.2) (layer "F.Cu") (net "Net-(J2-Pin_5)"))
 (segment (start 135.66 140.927969) (end 136.16 140.427969) (width 0.2) (layer "F.Cu") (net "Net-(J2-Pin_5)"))
 (segment (start 112.56 102.3) (end 108.06 106.800004) (width 0.2) (layer "F.Cu") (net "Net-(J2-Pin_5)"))
 (segment (start 111.791372 155.9) (end 122.328628 155.9) (width 0.2) (layer "F.Cu") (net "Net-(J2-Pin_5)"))
 (segment (start 135.66 142.568628) (end 135.66 140.927969) (width 0.2) (layer "F.Cu") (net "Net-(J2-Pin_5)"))
 (segment (start 136.16 140.427969) (end 136.16 137.54) (width 0.2) (layer "F.Cu") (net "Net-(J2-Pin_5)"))
 (segment (start 117.76 102.3) (end 112.56 102.3) (width 0.2) (layer "F.Cu") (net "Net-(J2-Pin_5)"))
 (segment (start 108.06 106.800004) (end 108.06 152.168628) (width 0.2) (layer "F.Cu") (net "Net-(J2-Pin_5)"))
 (segment (start 108.06 152.168628) (end 111.791372 155.9) (width 0.2) (layer "F.Cu") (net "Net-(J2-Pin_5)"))
 (segment (start 136.16 137.54) (end 137.56 136.14) (width 0.2) (layer "F.Cu") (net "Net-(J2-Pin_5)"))
 (segment (start 141.86 117.131372) (end 141.06 117.931373) (width 0.2) (layer "F.Cu") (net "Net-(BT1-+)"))
 (segment (start 191.76 71.434315) (end 185.225685 64.9) (width 0.2) (layer "F.Cu") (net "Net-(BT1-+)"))
 (segment (start 124.925686 106) (end 137.891371 106) (width 0.2) (layer "F.Cu") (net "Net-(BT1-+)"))
 (segment (start 124.71 119.2) (end 126.576346 119.2) (width 0.2) (layer "F.Cu") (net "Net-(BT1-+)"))
 (segment (start 122.96 107.965686) (end 124.925686 106) (width 0.2) (layer "F.Cu") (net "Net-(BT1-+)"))
 (segment (start 141.06 149.234314) (end 147.525687 155.7) (width 0.2) (layer "F.Cu") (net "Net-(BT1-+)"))
 (segment (start 141.06 117.931373) (end 141.06 149.234314) (width 0.2) (layer "F.Cu") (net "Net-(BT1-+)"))
 (segment (start 141.86 109.968629) (end 141.86 117.131372) (width 0.2) (layer "F.Cu") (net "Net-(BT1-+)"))
 (segment (start 179.46 64.9) (end 174.56 69.8) (width 0.2) (layer "F.Cu") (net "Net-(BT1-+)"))
 (segment (start 191.76 153.165684) (end 191.76 71.434315) (width 0.2) (layer "F.Cu") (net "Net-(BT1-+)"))
 (segment (start 126.576346 119.2) (end 127.25 118.526346) (width 0.2) (layer "F.Cu") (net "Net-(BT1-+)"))
 (segment (start 147.525687 155.7) (end 189.225685 155.7) (width 0.2) (layer "F.Cu") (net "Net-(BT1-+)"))
 (segment (start 127.25 117.573654) (end 122.96 113.283654) (width 0.2) (layer "F.Cu") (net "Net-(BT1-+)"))
 (segment (start 127.25 118.526346) (end 127.25 117.573654) (width 0.2) (layer "F.Cu") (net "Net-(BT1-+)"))
 (segment (start 122.96 113.283654) (end 122.96 107.965686) (width 0.2) (layer "F.Cu") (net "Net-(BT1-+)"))
 (segment (start 137.891371 106) (end 141.86 109.968629) (width 0.2) (layer "F.Cu") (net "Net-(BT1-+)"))
 (segment (start 185.225685 64.9) (end 179.46 64.9) (width 0.2) (layer "F.Cu") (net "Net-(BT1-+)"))
 (segment (start 123.56 118.05) (end 124.71 119.2) (width 0.2) (layer "F.Cu") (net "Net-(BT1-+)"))
 (segment (start 189.225685 155.7) (end 191.76 153.165684) (width 0.2) (layer "F.Cu") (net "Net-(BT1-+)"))
 (segment (start 147.36 156.1) (end 137.56 146.3) (width 0.2) (layer "F.Cu") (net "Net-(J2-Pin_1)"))
 (segment (start 181.691371 60.8) (end 192.16 71.268629) (width 0.2) (layer "F.Cu") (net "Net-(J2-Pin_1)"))
 (segment (start 120.6 64.3) (end 124.1 60.8) (width 0.2) (layer "F.Cu") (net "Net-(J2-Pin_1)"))
 (segment (start 124.1 60.8) (end 181.691371 60.8) (width 0.2) (layer "F.Cu") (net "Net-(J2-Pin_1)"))
 (segment (start 189.391371 156.1) (end 147.36 156.1) (width 0.2) (layer "F.Cu") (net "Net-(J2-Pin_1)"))
 (segment (start 192.16 71.268629) (end 192.16 153.331371) (width 0.2) (layer "F.Cu") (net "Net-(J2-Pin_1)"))
 (segment (start 192.16 153.331371) (end 189.391371 156.1) (width 0.2) (layer "F.Cu") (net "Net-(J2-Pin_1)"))
 (segment (start 136.99 142.37) (end 138.036346 142.37) (width 0.2) (layer "F.Cu") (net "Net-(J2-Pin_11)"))
 (segment (start 122.66 156.7) (end 136.99 142.37) (width 0.2) (layer "F.Cu") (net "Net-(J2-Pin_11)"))
 (segment (start 112.56 64.3) (end 107.26 69.6) (width 0.2) (layer "F.Cu") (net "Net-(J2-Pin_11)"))
 (segment (start 112.98 64.3) (end 112.56 64.3) (width 0.2) (layer "F.Cu") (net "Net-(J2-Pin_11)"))
 (segment (start 107.26 69.6) (end 107.26 152.5) (width 0.2) (layer "F.Cu") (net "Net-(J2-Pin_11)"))
 (segment (start 111.46 156.7) (end 122.66 156.7) (width 0.2) (layer "F.Cu") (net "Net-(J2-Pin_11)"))
 (segment (start 140.06 123.4) (end 137.56 120.9) (width 0.2) (layer "F.Cu") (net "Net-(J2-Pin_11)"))
 (segment (start 107.26 152.5) (end 111.46 156.7) (width 0.2) (layer "F.Cu") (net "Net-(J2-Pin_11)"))
 (segment (start 140.06 140.346346) (end 140.06 123.4) (width 0.2) (layer "F.Cu") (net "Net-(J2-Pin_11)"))
 (segment (start 138.036346 142.37) (end 140.06 140.346346) (width 0.2) (layer "F.Cu") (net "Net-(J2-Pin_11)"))
 (segment (start 137.09 124.83) (end 130.86 118.6) (width 0.2) (layer "F.Cu") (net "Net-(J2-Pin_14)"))
 (segment (start 107.66 69.765686) (end 107.66 152.334314) (width 0.2) (layer "F.Cu") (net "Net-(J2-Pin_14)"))
 (segment (start 138.71 125.503654) (end 138.036346 124.83) (width 0.2) (layer "F.Cu") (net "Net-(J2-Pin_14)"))
 (segment (start 114.606346 64.3) (end 113.456346 65.45) (width 0.2) (layer "F.Cu") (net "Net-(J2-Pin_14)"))
 (segment (start 113.456346 65.45) (end 111.975686 65.45) (width 0.2) (layer "F.Cu") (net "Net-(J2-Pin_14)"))
 (segment (start 138.71 139.156346) (end 138.71 125.503654) (width 0.2) (layer "F.Cu") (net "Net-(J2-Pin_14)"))
 (segment (start 111.625687 156.3) (end 122.494314 156.3) (width 0.2) (layer "F.Cu") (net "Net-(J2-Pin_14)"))
 (segment (start 107.66 152.334314) (end 111.625687 156.3) (width 0.2) (layer "F.Cu") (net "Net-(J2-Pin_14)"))
 (segment (start 136.06 141.093654) (end 137.323654 139.83) (width 0.2) (layer "F.Cu") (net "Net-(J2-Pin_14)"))
 (segment (start 137.323654 139.83) (end 138.036346 139.83) (width 0.2) (layer "F.Cu") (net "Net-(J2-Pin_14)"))
 (segment (start 122.494314 156.3) (end 136.06 142.734313) (width 0.2) (layer "F.Cu") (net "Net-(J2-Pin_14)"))
 (segment (start 130.86 118.6) (end 130.86 113.631372) (width 0.2) (layer "F.Cu") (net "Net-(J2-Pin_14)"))
 (segment (start 138.036346 139.83) (end 138.71 139.156346) (width 0.2) (layer "F.Cu") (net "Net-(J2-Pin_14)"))
 (segment (start 138.036346 124.83) (end 137.09 124.83) (width 0.2) (layer "F.Cu") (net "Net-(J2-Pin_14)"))
 (segment (start 136.58 112.3) (end 137.56 113.28) (width 0.2) (layer "F.Cu") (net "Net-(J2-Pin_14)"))
 (segment (start 130.86 113.631372) (end 132.191372 112.3) (width 0.2) (layer "F.Cu") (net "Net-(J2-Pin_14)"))
 (segment (start 111.975686 65.45) (end 107.66 69.765686) (width 0.2) (layer "F.Cu") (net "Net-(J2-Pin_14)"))
 (segment (start 115.52 64.3) (end 114.606346 64.3) (width 0.2) (layer "F.Cu") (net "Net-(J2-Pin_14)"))
 (segment (start 136.06 142.734313) (end 136.06 141.093654) (width 0.2) (layer "F.Cu") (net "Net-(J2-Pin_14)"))
 (segment (start 132.191372 112.3) (end 136.58 112.3) (width 0.2) (layer "F.Cu") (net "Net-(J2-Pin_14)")))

